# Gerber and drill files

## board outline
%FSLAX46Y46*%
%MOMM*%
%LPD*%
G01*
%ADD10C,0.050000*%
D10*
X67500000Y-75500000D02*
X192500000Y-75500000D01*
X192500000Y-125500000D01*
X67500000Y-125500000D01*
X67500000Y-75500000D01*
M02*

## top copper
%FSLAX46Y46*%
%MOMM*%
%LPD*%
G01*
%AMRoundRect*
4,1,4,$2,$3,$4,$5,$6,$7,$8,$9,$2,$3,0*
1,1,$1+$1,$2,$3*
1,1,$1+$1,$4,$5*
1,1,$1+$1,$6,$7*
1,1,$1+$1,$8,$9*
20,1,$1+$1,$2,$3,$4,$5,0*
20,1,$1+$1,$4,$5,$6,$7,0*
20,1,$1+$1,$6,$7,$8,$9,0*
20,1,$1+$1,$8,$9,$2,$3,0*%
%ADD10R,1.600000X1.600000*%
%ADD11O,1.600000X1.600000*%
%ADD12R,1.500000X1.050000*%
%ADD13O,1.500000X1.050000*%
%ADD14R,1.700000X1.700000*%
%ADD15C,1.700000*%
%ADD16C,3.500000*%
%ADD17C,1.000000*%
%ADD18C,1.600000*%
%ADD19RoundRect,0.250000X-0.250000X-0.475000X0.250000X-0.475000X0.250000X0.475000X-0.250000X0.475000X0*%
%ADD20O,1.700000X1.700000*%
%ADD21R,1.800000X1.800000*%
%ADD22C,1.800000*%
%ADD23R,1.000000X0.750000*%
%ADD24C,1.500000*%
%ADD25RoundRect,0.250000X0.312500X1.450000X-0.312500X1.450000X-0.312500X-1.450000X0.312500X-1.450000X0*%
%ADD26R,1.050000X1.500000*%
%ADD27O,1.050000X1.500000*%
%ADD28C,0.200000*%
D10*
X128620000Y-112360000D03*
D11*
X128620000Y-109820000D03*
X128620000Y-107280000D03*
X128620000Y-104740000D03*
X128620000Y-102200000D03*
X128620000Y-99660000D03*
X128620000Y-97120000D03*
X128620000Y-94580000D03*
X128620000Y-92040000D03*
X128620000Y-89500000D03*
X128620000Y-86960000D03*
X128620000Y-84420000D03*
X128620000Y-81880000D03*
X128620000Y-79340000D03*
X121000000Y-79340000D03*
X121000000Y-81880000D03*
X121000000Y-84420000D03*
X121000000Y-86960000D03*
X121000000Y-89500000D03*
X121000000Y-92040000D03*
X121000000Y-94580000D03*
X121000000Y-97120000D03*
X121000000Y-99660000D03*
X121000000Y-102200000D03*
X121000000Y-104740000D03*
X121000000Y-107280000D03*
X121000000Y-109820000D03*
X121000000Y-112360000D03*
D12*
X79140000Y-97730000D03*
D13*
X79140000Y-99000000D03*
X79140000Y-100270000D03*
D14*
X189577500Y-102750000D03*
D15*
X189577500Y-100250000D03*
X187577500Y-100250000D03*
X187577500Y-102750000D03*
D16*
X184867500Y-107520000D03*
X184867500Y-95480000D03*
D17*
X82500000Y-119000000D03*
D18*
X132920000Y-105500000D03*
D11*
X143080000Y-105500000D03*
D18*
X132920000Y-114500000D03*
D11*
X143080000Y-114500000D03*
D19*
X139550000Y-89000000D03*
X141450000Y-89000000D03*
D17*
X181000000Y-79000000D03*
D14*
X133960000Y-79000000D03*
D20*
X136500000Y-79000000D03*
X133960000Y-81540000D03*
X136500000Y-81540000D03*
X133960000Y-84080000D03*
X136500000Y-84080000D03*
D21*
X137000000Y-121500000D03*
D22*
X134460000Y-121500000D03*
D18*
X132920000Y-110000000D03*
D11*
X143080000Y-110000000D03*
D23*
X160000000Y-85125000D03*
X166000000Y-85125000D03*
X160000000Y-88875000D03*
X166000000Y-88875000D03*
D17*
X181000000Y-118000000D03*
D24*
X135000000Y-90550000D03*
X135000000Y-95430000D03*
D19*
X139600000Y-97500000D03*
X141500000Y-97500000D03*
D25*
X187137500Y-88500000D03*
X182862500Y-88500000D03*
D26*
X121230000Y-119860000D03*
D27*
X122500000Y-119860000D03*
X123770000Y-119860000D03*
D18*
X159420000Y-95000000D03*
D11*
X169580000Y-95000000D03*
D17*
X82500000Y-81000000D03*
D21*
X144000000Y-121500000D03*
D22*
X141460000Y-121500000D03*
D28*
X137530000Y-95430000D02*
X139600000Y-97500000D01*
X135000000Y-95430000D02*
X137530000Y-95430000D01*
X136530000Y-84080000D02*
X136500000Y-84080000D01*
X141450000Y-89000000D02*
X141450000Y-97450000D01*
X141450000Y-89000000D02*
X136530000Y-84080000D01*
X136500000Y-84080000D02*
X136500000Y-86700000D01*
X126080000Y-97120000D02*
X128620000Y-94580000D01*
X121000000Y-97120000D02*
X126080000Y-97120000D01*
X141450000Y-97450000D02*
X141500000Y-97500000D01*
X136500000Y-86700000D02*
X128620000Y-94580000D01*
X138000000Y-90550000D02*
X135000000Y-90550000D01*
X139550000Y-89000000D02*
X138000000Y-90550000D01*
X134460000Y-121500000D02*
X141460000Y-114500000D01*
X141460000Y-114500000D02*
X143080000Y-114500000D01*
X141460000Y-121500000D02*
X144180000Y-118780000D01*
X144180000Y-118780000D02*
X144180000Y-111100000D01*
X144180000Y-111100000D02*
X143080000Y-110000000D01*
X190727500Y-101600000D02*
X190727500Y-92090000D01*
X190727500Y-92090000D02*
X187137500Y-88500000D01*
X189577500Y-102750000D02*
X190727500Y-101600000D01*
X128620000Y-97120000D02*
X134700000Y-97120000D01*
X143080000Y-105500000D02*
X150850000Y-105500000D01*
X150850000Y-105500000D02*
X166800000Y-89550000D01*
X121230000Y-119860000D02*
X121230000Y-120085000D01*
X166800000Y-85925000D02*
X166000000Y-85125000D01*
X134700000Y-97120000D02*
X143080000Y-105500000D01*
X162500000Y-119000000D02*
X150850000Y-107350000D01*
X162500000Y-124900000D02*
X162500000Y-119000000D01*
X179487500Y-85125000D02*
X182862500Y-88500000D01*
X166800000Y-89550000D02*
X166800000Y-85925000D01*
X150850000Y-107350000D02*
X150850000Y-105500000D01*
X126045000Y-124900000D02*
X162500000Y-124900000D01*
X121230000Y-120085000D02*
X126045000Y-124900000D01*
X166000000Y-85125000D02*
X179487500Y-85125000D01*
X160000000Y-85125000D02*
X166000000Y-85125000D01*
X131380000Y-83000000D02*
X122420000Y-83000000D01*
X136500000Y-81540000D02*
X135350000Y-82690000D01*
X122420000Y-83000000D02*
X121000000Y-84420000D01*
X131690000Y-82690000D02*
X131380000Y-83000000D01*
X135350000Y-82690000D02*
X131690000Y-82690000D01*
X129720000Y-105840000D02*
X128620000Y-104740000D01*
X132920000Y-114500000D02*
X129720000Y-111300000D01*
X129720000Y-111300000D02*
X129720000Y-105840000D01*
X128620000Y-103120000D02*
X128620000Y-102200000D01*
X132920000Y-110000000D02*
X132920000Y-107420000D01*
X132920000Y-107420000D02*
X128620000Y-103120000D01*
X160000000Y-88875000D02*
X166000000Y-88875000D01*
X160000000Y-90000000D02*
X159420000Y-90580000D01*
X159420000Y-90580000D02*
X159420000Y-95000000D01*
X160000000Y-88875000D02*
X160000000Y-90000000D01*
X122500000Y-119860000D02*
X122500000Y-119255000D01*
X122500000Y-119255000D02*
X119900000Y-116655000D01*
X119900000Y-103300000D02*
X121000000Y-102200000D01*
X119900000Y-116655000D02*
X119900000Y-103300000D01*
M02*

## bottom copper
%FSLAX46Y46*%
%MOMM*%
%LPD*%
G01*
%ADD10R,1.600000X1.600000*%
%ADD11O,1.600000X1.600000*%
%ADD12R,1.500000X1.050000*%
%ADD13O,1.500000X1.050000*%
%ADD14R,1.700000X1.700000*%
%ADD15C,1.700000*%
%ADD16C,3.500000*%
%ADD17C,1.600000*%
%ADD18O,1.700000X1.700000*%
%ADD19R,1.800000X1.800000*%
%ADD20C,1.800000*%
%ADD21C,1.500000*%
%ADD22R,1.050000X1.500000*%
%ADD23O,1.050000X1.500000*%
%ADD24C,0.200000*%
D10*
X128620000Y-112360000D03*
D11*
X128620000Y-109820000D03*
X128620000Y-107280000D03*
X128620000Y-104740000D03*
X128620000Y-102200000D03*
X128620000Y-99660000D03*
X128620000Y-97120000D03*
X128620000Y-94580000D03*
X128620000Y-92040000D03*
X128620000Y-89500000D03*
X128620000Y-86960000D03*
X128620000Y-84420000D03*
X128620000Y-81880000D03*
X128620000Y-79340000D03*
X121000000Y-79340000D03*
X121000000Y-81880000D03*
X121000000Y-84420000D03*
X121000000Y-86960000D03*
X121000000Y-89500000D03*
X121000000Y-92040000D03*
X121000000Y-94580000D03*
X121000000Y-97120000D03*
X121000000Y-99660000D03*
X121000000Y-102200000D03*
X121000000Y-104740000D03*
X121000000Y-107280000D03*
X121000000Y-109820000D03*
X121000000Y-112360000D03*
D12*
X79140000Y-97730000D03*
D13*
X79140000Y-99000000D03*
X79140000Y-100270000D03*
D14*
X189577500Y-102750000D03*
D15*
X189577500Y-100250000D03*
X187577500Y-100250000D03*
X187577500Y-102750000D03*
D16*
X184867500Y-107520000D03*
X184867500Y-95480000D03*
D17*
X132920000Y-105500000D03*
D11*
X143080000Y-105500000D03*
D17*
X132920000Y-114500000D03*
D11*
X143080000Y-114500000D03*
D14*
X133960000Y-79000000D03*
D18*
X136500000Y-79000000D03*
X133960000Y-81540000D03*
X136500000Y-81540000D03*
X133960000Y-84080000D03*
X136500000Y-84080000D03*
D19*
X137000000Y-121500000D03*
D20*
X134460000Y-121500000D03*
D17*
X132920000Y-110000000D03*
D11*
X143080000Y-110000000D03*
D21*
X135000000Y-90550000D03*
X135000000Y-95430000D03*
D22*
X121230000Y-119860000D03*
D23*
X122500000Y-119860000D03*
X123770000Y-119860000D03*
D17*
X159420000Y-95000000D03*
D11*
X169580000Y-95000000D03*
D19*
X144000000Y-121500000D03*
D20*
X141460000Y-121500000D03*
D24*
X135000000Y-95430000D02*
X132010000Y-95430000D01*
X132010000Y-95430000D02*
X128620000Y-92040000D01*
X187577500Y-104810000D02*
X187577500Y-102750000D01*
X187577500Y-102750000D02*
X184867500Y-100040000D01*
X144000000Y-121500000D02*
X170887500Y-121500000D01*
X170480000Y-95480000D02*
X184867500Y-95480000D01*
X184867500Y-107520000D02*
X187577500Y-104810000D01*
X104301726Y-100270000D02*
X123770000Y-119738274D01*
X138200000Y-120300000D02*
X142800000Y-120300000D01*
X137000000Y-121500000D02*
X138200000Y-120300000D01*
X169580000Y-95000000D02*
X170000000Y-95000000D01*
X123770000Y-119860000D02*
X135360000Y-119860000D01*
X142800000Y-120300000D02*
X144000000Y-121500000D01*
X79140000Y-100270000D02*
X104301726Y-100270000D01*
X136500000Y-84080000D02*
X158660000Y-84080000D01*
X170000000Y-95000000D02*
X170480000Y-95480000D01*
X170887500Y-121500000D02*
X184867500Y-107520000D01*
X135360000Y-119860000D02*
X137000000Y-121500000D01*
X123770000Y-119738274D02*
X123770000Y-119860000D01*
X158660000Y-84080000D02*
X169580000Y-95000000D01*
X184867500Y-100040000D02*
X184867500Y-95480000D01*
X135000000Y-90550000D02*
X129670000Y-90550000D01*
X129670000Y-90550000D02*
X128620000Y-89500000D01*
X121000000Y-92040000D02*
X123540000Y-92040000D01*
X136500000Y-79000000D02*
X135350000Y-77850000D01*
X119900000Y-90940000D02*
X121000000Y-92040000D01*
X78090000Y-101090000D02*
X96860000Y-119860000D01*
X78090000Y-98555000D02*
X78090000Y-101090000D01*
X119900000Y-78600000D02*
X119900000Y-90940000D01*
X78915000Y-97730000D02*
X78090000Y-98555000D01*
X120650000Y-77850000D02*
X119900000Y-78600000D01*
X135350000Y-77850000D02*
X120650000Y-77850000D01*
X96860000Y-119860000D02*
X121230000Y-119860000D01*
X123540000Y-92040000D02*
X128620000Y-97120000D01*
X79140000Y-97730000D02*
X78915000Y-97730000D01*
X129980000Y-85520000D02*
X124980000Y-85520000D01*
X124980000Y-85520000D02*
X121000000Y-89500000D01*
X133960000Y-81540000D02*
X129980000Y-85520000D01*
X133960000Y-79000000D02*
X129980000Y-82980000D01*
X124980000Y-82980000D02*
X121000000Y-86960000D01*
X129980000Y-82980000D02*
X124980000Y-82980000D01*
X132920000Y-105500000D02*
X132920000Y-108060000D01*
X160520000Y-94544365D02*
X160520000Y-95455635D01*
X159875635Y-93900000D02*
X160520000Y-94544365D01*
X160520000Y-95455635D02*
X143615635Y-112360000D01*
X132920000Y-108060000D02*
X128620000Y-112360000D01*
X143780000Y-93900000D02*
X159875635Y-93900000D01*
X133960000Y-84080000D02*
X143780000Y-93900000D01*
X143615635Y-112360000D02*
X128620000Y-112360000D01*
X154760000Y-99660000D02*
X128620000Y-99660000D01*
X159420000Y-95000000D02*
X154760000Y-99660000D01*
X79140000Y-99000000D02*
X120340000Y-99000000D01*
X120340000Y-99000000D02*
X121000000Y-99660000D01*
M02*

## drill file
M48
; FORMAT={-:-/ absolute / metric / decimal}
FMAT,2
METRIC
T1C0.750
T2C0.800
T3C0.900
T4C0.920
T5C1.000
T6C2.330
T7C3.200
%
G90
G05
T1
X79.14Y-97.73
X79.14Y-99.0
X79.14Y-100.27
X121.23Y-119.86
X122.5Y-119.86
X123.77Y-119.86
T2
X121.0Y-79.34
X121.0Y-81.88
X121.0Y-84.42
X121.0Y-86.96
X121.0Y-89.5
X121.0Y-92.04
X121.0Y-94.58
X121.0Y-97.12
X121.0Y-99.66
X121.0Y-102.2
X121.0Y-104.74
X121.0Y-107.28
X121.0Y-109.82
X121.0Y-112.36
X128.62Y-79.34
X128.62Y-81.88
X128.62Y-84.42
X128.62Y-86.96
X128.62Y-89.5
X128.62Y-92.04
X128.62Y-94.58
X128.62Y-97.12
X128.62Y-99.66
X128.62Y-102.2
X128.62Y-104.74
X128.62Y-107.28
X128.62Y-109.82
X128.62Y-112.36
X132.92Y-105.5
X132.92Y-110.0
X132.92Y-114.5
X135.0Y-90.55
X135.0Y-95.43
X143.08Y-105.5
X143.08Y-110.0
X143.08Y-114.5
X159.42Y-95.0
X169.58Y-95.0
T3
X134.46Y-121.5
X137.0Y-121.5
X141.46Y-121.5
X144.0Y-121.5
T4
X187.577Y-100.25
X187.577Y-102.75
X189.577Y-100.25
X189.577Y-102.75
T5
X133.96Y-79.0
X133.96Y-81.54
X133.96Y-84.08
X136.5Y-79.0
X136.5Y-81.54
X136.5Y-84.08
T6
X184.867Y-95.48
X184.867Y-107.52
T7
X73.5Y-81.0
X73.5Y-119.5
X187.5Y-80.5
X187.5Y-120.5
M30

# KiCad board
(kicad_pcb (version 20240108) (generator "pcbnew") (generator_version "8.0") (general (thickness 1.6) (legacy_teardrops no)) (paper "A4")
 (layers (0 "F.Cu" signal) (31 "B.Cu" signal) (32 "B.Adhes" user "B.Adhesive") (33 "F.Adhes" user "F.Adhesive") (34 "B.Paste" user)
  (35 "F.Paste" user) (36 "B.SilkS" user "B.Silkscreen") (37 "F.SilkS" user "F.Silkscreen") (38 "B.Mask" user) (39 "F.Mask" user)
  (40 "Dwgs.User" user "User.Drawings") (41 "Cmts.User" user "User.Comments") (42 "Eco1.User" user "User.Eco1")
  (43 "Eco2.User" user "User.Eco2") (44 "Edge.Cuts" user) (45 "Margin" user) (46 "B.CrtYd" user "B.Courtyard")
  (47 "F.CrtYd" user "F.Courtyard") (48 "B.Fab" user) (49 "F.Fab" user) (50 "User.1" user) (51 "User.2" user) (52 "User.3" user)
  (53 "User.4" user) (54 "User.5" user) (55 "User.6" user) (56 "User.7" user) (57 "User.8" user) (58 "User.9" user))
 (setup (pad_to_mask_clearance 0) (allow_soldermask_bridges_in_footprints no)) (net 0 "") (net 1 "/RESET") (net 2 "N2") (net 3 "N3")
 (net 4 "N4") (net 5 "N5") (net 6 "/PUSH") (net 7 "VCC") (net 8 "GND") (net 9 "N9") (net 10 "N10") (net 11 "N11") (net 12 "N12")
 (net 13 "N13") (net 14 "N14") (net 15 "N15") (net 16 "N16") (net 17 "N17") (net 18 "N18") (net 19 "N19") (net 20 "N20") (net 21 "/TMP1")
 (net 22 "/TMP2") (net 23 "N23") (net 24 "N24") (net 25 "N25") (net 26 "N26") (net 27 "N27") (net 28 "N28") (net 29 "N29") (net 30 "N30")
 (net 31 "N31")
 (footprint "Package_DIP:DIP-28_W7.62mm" (layer "F.Cu") (at 128.62 112.36 180)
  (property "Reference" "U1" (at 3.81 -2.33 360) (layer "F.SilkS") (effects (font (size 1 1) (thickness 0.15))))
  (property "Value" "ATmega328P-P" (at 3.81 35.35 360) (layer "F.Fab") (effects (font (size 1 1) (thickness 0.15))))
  (pad "1" thru_hole rect (at 0 0 180) (size 1.6 1.6) (drill 0.8) (layers "*.Cu" "*.Mask") (remove_unused_layers no) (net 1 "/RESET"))
  (pad "2" thru_hole oval (at 0 2.54 180) (size 1.6 1.6) (drill 0.8) (layers "*.Cu" "*.Mask") (remove_unused_layers no) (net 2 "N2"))
  (pad "3" thru_hole oval (at 0 5.08 180) (size 1.6 1.6) (drill 0.8) (layers "*.Cu" "*.Mask") (remove_unused_layers no) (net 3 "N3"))
  (pad "4" thru_hole oval (at 0 7.62 180) (size 1.6 1.6) (drill 0.8) (layers "*.Cu" "*.Mask") (remove_unused_layers no) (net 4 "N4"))
  (pad "5" thru_hole oval (at 0 10.16 180) (size 1.6 1.6) (drill 0.8) (layers "*.Cu" "*.Mask") (remove_unused_layers no) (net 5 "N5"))
  (pad "6" thru_hole oval (at 0 12.7 180) (size 1.6 1.6) (drill 0.8) (layers "*.Cu" "*.Mask") (remove_unused_layers no) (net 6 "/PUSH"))
  (pad "7" thru_hole oval (at 0 15.24 180) (size 1.6 1.6) (drill 0.8) (layers "*.Cu" "*.Mask") (remove_unused_layers no) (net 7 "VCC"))
  (pad "8" thru_hole oval (at 0 17.78 180) (size 1.6 1.6) (drill 0.8) (layers "*.Cu" "*.Mask") (remove_unused_layers no) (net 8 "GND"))
  (pad "9" thru_hole oval (at 0 20.32 180) (size 1.6 1.6) (drill 0.8) (layers "*.Cu" "*.Mask") (remove_unused_layers no) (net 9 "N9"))
  (pad "10" thru_hole oval (at 0 22.86 180) (size 1.6 1.6) (drill 0.8) (layers "*.Cu" "*.Mask") (remove_unused_layers no) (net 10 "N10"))
  (pad "11" thru_hole oval (at 0 25.4 180) (size 1.6 1.6) (drill 0.8) (layers "*.Cu" "*.Mask") (remove_unused_layers no) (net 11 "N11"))
  (pad "12" thru_hole oval (at 0 27.94 180) (size 1.6 1.6) (drill 0.8) (layers "*.Cu" "*.Mask") (remove_unused_layers no) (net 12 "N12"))
  (pad "13" thru_hole oval (at 0 30.48 180) (size 1.6 1.6) (drill 0.8) (layers "*.Cu" "*.Mask") (remove_unused_layers no) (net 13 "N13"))
  (pad "14" thru_hole oval (at 0 33.02 180) (size 1.6 1.6) (drill 0.8) (layers "*.Cu" "*.Mask") (remove_unused_layers no) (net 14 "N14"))
  (pad "15" thru_hole oval (at 7.62 33.02 180) (size 1.6 1.6) (drill 0.8) (layers "*.Cu" "*.Mask") (remove_unused_layers no) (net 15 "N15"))
  (pad "16" thru_hole oval (at 7.62 30.48 180) (size 1.6 1.6) (drill 0.8) (layers "*.Cu" "*.Mask") (remove_unused_layers no) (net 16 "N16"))
  (pad "17" thru_hole oval (at 7.62 27.94 180) (size 1.6 1.6) (drill 0.8) (layers "*.Cu" "*.Mask") (remove_unused_layers no) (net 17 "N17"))
  (pad "18" thru_hole oval (at 7.62 25.4 180) (size 1.6 1.6) (drill 0.8) (layers "*.Cu" "*.Mask") (remove_unused_layers no) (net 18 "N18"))
  (pad "19" thru_hole oval (at 7.62 22.86 180) (size 1.6 1.6) (drill 0.8) (layers "*.Cu" "*.Mask") (remove_unused_layers no) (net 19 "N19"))
  (pad "20" thru_hole oval (at 7.62 20.32 180) (size 1.6 1.6) (drill 0.8) (layers "*.Cu" "*.Mask") (remove_unused_layers no) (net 7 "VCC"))
  (pad "21" thru_hole oval (at 7.62 17.78 180) (size 1.6 1.6) (drill 0.8) (layers "*.Cu" "*.Mask") (remove_unused_layers no) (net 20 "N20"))
  (pad "22" thru_hole oval (at 7.62 15.24 180) (size 1.6 1.6) (drill 0.8) (layers "*.Cu" "*.Mask") (remove_unused_layers no) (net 8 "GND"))
  (pad "23" thru_hole oval (at 7.62 12.7 180) (size 1.6 1.6) (drill 0.8) (layers "*.Cu" "*.Mask") (remove_unused_layers no) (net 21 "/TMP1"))
  (pad "24" thru_hole oval (at 7.62 10.16 180) (size 1.6 1.6) (drill 0.8) (layers "*.Cu" "*.Mask") (remove_unused_layers no)
   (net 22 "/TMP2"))
  (pad "25" thru_hole oval (at 7.62 7.62 180) (size 1.6 1.6) (drill 0.8) (layers "*.Cu" "*.Mask") (remove_unused_layers no) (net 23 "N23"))
  (pad "26" thru_hole oval (at 7.62 5.08 180) (size 1.6 1.6) (drill 0.8) (layers "*.Cu" "*.Mask") (remove_unused_layers no) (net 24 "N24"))
  (pad "27" thru_hole oval (at 7.62 2.54 180) (size 1.6 1.6) (drill 0.8) (layers "*.Cu" "*.Mask") (remove_unused_layers no) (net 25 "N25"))
  (pad "28" thru_hole oval (at 7.62 0 180) (size 1.6 1.6) (drill 0.8) (layers "*.Cu" "*.Mask") (remove_unused_layers no) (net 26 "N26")))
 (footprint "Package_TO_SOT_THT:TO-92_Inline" (layer "F.Cu") (at 79.14 97.73 -90)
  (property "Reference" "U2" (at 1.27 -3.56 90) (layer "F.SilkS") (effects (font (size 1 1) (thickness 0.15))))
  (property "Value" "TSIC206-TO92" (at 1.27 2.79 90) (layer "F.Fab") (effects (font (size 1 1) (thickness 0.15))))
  (pad "1" thru_hole rect (at 0 0 270) (size 1.05 1.5) (drill 0.75) (layers "*.Cu" "*.Mask") (remove_unused_layers no) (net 7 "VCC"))
  (pad "2" thru_hole oval (at 1.27 0 270) (size 1.05 1.5) (drill 0.75) (layers "*.Cu" "*.Mask") (remove_unused_layers no) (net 21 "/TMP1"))
  (pad "3" thru_hole oval (at 2.54 0 270) (size 1.05 1.5) (drill 0.75) (layers "*.Cu" "*.Mask") (remove_unused_layers no) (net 8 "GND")))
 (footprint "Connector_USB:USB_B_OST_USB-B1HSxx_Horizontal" (layer "F.Cu") (at 189.5775 102.75 180)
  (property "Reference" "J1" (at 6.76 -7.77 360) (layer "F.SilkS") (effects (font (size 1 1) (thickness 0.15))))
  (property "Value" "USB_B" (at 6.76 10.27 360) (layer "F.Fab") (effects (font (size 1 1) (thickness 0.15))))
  (pad "1" thru_hole rect (at 0 0 180) (size 1.7 1.7) (drill 0.92) (layers "*.Cu" "*.Mask") (remove_unused_layers no) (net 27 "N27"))
  (pad "2" thru_hole circle (at 0 2.5 180) (size 1.7 1.7) (drill 0.92) (layers "*.Cu" "*.Mask") (remove_unused_layers no) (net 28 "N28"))
  (pad "3" thru_hole circle (at 2 2.5 180) (size 1.7 1.7) (drill 0.92) (layers "*.Cu" "*.Mask") (remove_unused_layers no) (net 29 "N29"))
  (pad "4" thru_hole circle (at 2 0 180) (size 1.7 1.7) (drill 0.92) (layers "*.Cu" "*.Mask") (remove_unused_layers no) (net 8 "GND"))
  (pad "5" thru_hole circle (at 4.71 -4.77 180) (size 3.5 3.5) (drill 2.33) (layers "*.Cu" "*.Mask") (remove_unused_layers no) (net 8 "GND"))
  (pad "5" thru_hole circle (at 4.71 7.27 180) (size 3.5 3.5) (drill 2.33) (layers "*.Cu" "*.Mask") (remove_unused_layers no) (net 8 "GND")))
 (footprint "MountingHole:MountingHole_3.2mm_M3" (layer "F.Cu") (at 73.5 81)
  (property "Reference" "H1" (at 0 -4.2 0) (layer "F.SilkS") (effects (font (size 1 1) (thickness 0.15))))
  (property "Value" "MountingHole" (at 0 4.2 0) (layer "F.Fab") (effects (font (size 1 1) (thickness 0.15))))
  (pad "" np_thru_hole circle (at 0 0) (size 3.2 3.2) (drill 3.2) (layers "*.Cu" "*.Mask")))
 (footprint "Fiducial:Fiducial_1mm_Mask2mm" (layer "F.Cu") (at 82.5 119)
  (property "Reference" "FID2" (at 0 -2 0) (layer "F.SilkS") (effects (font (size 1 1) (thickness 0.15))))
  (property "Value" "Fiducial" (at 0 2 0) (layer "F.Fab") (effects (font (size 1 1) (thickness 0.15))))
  (pad "" smd circle (at 0 0) (size 1 1) (layers "F.Cu" "F.Mask") (solder_mask_margin 0.5) (clearance 0.5)))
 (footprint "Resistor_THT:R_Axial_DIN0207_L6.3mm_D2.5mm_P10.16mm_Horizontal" (layer "F.Cu") (at 132.92 105.5)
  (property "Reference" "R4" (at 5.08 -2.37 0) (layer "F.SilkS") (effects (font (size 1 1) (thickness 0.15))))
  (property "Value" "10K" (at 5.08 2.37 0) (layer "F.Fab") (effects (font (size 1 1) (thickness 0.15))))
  (pad "1" thru_hole circle (at 0 0) (size 1.6 1.6) (drill 0.8) (layers "*.Cu" "*.Mask") (remove_unused_layers no) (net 1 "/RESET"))
  (pad "2" thru_hole oval (at 10.16 0) (size 1.6 1.6) (drill 0.8) (layers "*.Cu" "*.Mask") (remove_unused_layers no) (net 7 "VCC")))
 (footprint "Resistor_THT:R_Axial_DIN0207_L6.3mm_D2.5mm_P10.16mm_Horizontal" (layer "F.Cu") (at 132.92 114.5)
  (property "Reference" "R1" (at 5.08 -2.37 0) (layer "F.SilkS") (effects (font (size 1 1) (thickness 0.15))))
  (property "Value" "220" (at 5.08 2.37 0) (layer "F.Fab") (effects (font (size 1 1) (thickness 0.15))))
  (pad "1" thru_hole circle (at 0 0) (size 1.6 1.6) (drill 0.8) (layers "*.Cu" "*.Mask") (remove_unused_layers no) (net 4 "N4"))
  (pad "2" thru_hole oval (at 10.16 0) (size 1.6 1.6) (drill 0.8) (layers "*.Cu" "*.Mask") (remove_unused_layers no) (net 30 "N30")))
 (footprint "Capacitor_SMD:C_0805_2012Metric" (layer "F.Cu") (at 140.5 89)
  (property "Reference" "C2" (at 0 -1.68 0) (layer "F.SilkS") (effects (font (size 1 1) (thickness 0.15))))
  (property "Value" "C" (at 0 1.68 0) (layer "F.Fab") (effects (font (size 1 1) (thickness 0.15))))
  (pad "1" smd roundrect (at -0.95 0) (size 1 1.45) (layers "F.Cu" "F.Paste" "F.Mask") (roundrect_rratio 0.25) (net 10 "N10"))
  (pad "2" smd roundrect (at 0.95 0) (size 1 1.45) (layers "F.Cu" "F.Paste" "F.Mask") (roundrect_rratio 0.25) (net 8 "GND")))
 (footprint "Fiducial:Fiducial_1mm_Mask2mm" (layer "F.Cu") (at 181 79)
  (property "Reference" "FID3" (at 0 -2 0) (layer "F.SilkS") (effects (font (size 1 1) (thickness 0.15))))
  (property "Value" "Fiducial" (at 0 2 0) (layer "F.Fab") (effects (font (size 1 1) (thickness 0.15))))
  (pad "" smd circle (at 0 0) (size 1 1) (layers "F.Cu" "F.Mask") (solder_mask_margin 0.5) (clearance 0.5)))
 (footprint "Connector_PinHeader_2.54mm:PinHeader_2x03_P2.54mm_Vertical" (layer "F.Cu") (at 133.96 79)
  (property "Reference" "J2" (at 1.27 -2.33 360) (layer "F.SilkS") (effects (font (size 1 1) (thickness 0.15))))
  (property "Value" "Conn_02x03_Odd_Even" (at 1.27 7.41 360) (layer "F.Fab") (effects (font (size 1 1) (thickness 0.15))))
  (pad "1" thru_hole rect (at 0 0) (size 1.7 1.7) (drill 1) (layers "*.Cu" "*.Mask") (remove_unused_layers no) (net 18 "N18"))
  (pad "2" thru_hole oval (at 2.54 0) (size 1.7 1.7) (drill 1) (layers "*.Cu" "*.Mask") (remove_unused_layers no) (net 7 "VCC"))
  (pad "3" thru_hole oval (at 0 2.54) (size 1.7 1.7) (drill 1) (layers "*.Cu" "*.Mask") (remove_unused_layers no) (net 19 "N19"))
  (pad "4" thru_hole oval (at 2.54 2.54) (size 1.7 1.7) (drill 1) (layers "*.Cu" "*.Mask") (remove_unused_layers no) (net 17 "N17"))
  (pad "5" thru_hole oval (at 0 5.08) (size 1.7 1.7) (drill 1) (layers "*.Cu" "*.Mask") (remove_unused_layers no) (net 1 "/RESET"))
  (pad "6" thru_hole oval (at 2.54 5.08) (size 1.7 1.7) (drill 1) (layers "*.Cu" "*.Mask") (remove_unused_layers no) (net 8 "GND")))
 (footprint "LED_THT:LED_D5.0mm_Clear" (layer "F.Cu") (at 137 121.5 180)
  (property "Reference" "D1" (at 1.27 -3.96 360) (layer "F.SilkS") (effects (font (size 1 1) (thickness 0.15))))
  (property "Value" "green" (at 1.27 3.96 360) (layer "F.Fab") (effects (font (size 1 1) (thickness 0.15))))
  (pad "1" thru_hole rect (at 0 0 180) (size 1.8 1.8) (drill 0.9) (layers "*.Cu" "*.Mask") (remove_unused_layers no) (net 8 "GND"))
  (pad "2" thru_hole circle (at 2.54 0 180) (size 1.8 1.8) (drill 0.9) (layers "*.Cu" "*.Mask") (remove_unused_layers no) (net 30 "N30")))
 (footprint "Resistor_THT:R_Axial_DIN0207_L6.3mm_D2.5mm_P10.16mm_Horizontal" (layer "F.Cu") (at 132.92 110)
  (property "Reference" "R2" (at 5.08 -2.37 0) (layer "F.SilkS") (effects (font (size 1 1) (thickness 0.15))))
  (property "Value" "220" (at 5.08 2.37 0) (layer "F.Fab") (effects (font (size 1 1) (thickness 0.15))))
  (pad "1" thru_hole circle (at 0 0) (size 1.6 1.6) (drill 0.8) (layers "*.Cu" "*.Mask") (remove_unused_layers no) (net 5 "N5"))
  (pad "2" thru_hole oval (at 10.16 0) (size 1.6 1.6) (drill 0.8) (layers "*.Cu" "*.Mask") (remove_unused_layers no) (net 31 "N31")))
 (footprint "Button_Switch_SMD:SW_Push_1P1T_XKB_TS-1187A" (layer "F.Cu") (at 163 87)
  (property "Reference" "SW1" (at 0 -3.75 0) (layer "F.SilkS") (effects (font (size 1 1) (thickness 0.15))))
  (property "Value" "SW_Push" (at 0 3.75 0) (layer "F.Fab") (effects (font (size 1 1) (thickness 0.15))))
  (pad "1" smd rect (at -3 -1.875) (size 1 0.75) (layers "F.Cu" "F.Paste" "F.Mask") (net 7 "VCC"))
  (pad "1" smd rect (at 3 -1.875) (size 1 0.75) (layers "F.Cu" "F.Paste" "F.Mask") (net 7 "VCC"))
  (pad "2" smd rect (at -3 1.875) (size 1 0.75) (layers "F.Cu" "F.Paste" "F.Mask") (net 6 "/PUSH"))
  (pad "2" smd rect (at 3 1.875) (size 1 0.75) (layers "F.Cu" "F.Paste" "F.Mask") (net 6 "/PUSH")))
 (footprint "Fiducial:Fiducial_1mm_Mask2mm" (layer "F.Cu") (at 181 118)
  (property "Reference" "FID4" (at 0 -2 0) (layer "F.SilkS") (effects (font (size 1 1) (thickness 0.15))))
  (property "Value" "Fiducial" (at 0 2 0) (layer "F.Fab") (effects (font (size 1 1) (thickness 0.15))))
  (pad "" smd circle (at 0 0) (size 1 1) (layers "F.Cu" "F.Mask") (solder_mask_margin 0.5) (clearance 0.5)))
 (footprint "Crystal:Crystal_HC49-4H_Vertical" (layer "F.Cu") (at 135 90.55 -90)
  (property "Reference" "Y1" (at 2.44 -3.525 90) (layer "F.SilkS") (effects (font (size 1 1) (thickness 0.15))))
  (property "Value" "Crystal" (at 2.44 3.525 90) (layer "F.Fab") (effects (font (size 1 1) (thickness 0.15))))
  (pad "1" thru_hole circle (at 0 0 270) (size 1.5 1.5) (drill 0.8) (layers "*.Cu" "*.Mask") (remove_unused_layers no) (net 10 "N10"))
  (pad "2" thru_hole circle (at 4.88 0 270) (size 1.5 1.5) (drill 0.8) (layers "*.Cu" "*.Mask") (remove_unused_layers no) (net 9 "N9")))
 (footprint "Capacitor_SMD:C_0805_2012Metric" (layer "F.Cu") (at 140.55 97.5)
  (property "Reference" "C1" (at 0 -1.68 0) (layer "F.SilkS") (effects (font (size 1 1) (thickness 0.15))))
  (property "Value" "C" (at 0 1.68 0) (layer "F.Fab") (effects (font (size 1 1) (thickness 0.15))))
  (pad "1" smd roundrect (at -0.95 0) (size 1 1.45) (layers "F.Cu" "F.Paste" "F.Mask") (roundrect_rratio 0.25) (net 9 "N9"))
  (pad "2" smd roundrect (at 0.95 0) (size 1 1.45) (layers "F.Cu" "F.Paste" "F.Mask") (roundrect_rratio 0.25) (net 8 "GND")))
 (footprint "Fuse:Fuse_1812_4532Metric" (layer "F.Cu") (at 185 88.5 180)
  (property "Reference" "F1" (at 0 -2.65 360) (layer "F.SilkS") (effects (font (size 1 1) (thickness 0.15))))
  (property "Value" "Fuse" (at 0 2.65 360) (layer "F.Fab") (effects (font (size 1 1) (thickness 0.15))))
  (pad "1" smd roundrect (at -2.1375 0 180) (size 1.125 3.4) (layers "F.Cu" "F.Paste" "F.Mask") (roundrect_rratio 0.222222) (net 27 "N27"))
  (pad "2" smd roundrect (at 2.1375 0 180) (size 1.125 3.4) (layers "F.Cu" "F.Paste" "F.Mask") (roundrect_rratio 0.222222) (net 7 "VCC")))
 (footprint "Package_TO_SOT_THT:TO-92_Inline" (layer "F.Cu") (at 121.23 119.86)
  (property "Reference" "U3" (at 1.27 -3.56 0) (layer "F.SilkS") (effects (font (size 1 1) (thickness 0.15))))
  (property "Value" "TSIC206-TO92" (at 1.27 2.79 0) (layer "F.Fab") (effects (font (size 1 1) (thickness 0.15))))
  (pad "1" thru_hole rect (at 0 0) (size 1.05 1.5) (drill 0.75) (layers "*.Cu" "*.Mask") (remove_unused_layers no) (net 7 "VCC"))
  (pad "2" thru_hole oval (at 1.27 0) (size 1.05 1.5) (drill 0.75) (layers "*.Cu" "*.Mask") (remove_unused_layers no) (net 22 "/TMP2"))
  (pad "3" thru_hole oval (at 2.54 0) (size 1.05 1.5) (drill 0.75) (layers "*.Cu" "*.Mask") (remove_unused_layers no) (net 8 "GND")))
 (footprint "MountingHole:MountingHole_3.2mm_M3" (layer "F.Cu") (at 73.5 119.5)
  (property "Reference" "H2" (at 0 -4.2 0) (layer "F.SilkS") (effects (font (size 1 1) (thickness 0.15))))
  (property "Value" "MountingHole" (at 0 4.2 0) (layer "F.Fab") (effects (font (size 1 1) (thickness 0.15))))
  (pad "" np_thru_hole circle (at 0 0) (size 3.2 3.2) (drill 3.2) (layers "*.Cu" "*.Mask")))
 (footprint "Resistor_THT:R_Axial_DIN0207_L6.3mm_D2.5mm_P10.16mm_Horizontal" (layer "F.Cu") (at 159.42 95)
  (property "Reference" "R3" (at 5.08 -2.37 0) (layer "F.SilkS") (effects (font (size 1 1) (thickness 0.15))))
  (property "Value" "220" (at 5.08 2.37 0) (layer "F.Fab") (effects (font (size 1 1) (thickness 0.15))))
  (pad "1" thru_hole circle (at 0 0) (size 1.6 1.6) (drill 0.8) (layers "*.Cu" "*.Mask") (remove_unused_layers no) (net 6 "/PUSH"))
  (pad "2" thru_hole oval (at 10.16 0) (size 1.6 1.6) (drill 0.8) (layers "*.Cu" "*.Mask") (remove_unused_layers no) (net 8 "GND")))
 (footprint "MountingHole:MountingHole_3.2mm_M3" (layer "F.Cu") (at 187.5 80.5)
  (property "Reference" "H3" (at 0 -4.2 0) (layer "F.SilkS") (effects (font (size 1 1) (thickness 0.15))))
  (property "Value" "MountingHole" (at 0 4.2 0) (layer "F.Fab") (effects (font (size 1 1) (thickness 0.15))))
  (pad "" np_thru_hole circle (at 0 0) (size 3.2 3.2) (drill 3.2) (layers "*.Cu" "*.Mask")))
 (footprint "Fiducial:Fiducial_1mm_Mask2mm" (layer "F.Cu") (at 82.5 81)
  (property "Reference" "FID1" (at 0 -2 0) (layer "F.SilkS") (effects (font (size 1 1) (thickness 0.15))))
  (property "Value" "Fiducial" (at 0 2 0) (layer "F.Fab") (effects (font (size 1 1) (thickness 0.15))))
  (pad "" smd circle (at 0 0) (size 1 1) (layers "F.Cu" "F.Mask") (solder_mask_margin 0.5) (clearance 0.5)))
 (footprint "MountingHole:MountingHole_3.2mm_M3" (layer "F.Cu") (at 187.5 120.5)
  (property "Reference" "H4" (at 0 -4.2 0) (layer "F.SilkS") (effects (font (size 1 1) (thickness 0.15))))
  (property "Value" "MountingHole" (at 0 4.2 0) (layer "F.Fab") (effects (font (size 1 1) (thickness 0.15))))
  (pad "" np_thru_hole circle (at 0 0) (size 3.2 3.2) (drill 3.2) (layers "*.Cu" "*.Mask")))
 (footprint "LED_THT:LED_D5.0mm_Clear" (layer "F.Cu") (at 144 121.5 180)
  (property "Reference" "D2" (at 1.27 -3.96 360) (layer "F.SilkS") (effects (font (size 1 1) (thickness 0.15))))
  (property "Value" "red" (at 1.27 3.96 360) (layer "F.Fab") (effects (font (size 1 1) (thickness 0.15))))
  (pad "1" thru_hole rect (at 0 0 180) (size 1.8 1.8) (drill 0.9) (layers "*.Cu" "*.Mask") (remove_unused_layers no) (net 8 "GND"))
  (pad "2" thru_hole circle (at 2.54 0 180) (size 1.8 1.8) (drill 0.9) (layers "*.Cu" "*.Mask") (remove_unused_layers no) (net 31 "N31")))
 (gr_rect (start 67.5 75.5) (end 192.5 125.5) (stroke (width 0.05) (type default)) (fill none) (layer "Edge.Cuts"))
 (segment (start 137.53 95.43) (end 139.6 97.5) (width 0.2) (layer "F.Cu") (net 9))
 (segment (start 135 95.43) (end 137.53 95.43) (width 0.2) (layer "F.Cu") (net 9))
 (segment (start 135 95.43) (end 132.01 95.43) (width 0.2) (layer "B.Cu") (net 9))
 (segment (start 132.01 95.43) (end 128.62 92.04) (width 0.2) (layer "B.Cu") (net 9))
 (segment (start 136.53 84.08) (end 136.5 84.08) (width 0.2) (layer "F.Cu") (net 8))
 (segment (start 141.45 89) (end 141.45 97.45) (width 0.2) (layer "F.Cu") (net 8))
 (segment (start 141.45 89) (end 136.53 84.08) (width 0.2) (layer "F.Cu") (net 8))
 (segment (start 136.5 84.08) (end 136.5 86.7) (width 0.2) (layer "F.Cu") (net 8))
 (segment (start 126.08 97.12) (end 128.62 94.58) (width 0.2) (layer "F.Cu") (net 8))
 (segment (start 121 97.12) (end 126.08 97.12) (width 0.2) (layer "F.Cu") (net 8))
 (segment (start 141.45 97.45) (end 141.5 97.5) (width 0.2) (layer "F.Cu") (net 8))
 (segment (start 136.5 86.7) (end 128.62 94.58) (width 0.2) (layer "F.Cu") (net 8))
 (segment (start 187.5775 104.81) (end 187.5775 102.75) (width 0.2) (layer "B.Cu") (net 8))
 (segment (start 187.5775 102.75) (end 184.8675 100.04) (width 0.2) (layer "B.Cu") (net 8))
 (segment (start 144 121.5) (end 170.8875 121.5) (width 0.2) (layer "B.Cu") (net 8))
 (segment (start 170.48 95.48) (end 184.8675 95.48) (width 0.2) (layer "B.Cu") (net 8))
 (segment (start 184.8675 107.52) (end 187.5775 104.81) (width 0.2) (layer "B.Cu") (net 8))
 (segment (start 104.301726 100.27) (end 123.77 119.738274) (width 0.2) (layer "B.Cu") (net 8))
 (segment (start 138.2 120.3) (end 142.8 120.3) (width 0.2) (layer "B.Cu") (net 8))
 (segment (start 137 121.5) (end 138.2 120.3) (width 0.2) (layer "B.Cu") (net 8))
 (segment (start 169.58 95) (end 170 95) (width 0.2) (layer "B.Cu") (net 8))
 (segment (start 123.77 119.86) (end 135.36 119.86) (width 0.2) (layer "B.Cu") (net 8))
 (segment (start 142.8 120.3) (end 144 121.5) (width 0.2) (layer "B.Cu") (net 8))
 (segment (start 79.14 100.27) (end 104.301726 100.27) (width 0.2) (layer "B.Cu") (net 8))
 (segment (start 136.5 84.08) (end 158.66 84.08) (width 0.2) (layer "B.Cu") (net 8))
 (segment (start 170 95) (end 170.48 95.48) (width 0.2) (layer "B.Cu") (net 8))
 (segment (start 170.8875 121.5) (end 184.8675 107.52) (width 0.2) (layer "B.Cu") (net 8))
 (segment (start 135.36 119.86) (end 137 121.5) (width 0.2) (layer "B.Cu") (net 8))
 (segment (start 123.77 119.738274) (end 123.77 119.86) (width 0.2) (layer "B.Cu") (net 8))
 (segment (start 158.66 84.08) (end 169.58 95) (width 0.2) (layer "B.Cu") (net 8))
 (segment (start 184.8675 100.04) (end 184.8675 95.48) (width 0.2) (layer "B.Cu") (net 8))
 (segment (start 138 90.55) (end 135 90.55) (width 0.2) (layer "F.Cu") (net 10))
 (segment (start 139.55 89) (end 138 90.55) (width 0.2) (layer "F.Cu") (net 10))
 (segment (start 135 90.55) (end 129.67 90.55) (width 0.2) (layer "B.Cu") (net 10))
 (segment (start 129.67 90.55) (end 128.62 89.5) (width 0.2) (layer "B.Cu") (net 10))
 (segment (start 134.46 121.5) (end 141.46 114.5) (width 0.2) (layer "F.Cu") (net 30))
 (segment (start 141.46 114.5) (end 143.08 114.5) (width 0.2) (layer "F.Cu") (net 30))
 (segment (start 141.46 121.5) (end 144.18 118.78) (width 0.2) (layer "F.Cu") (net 31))
 (segment (start 144.18 118.78) (end 144.18 111.1) (width 0.2) (layer "F.Cu") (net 31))
 (segment (start 144.18 111.1) (end 143.08 110) (width 0.2) (layer "F.Cu") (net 31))
 (segment (start 190.7275 101.6) (end 190.7275 92.09) (width 0.2) (layer "F.Cu") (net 27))
 (segment (start 190.7275 92.09) (end 187.1375 88.5) (width 0.2) (layer "F.Cu") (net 27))
 (segment (start 189.5775 102.75) (end 190.7275 101.6) (width 0.2) (layer "F.Cu") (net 27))
 (segment (start 128.62 97.12) (end 134.7 97.12) (width 0.2) (layer "F.Cu") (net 7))
 (segment (start 143.08 105.5) (end 150.85 105.5) (width 0.2) (layer "F.Cu") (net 7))
 (segment (start 150.85 105.5) (end 166.8 89.55) (width 0.2) (layer "F.Cu") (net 7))
 (segment (start 121.23 119.86) (end 121.23 120.085) (width 0.2) (layer "F.Cu") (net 7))
 (segment (start 166.8 85.925) (end 166 85.125) (width 0.2) (layer "F.Cu") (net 7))
 (segment (start 134.7 97.12) (end 143.08 105.5) (width 0.2) (layer "F.Cu") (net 7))
 (segment (start 162.5 119) (end 150.85 107.35) (width 0.2) (layer "F.Cu") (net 7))
 (segment (start 162.5 124.9) (end 162.5 119) (width 0.2) (layer "F.Cu") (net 7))
 (segment (start 179.4875 85.125) (end 182.8625 88.5) (width 0.2) (layer "F.Cu") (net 7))
 (segment (start 166.8 89.55) (end 166.8 85.925) (width 0.2) (layer "F.Cu") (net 7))
 (segment (start 150.85 107.35) (end 150.85 105.5) (width 0.2) (layer "F.Cu") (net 7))
 (segment (start 126.045 124.9) (end 162.5 124.9) (width 0.2) (layer "F.Cu") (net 7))
 (segment (start 121.23 120.085) (end 126.045 124.9) (width 0.2) (layer "F.Cu") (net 7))
 (segment (start 166 85.125) (end 179.4875 85.125) (width 0.2) (layer "F.Cu") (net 7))
 (segment (start 160 85.125) (end 166 85.125) (width 0.2) (layer "F.Cu") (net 7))
 (segment (start 121 92.04) (end 123.54 92.04) (width 0.2) (layer "B.Cu") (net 7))
 (segment (start 136.5 79) (end 135.35 77.85) (width 0.2) (layer "B.Cu") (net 7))
 (segment (start 119.9 90.94) (end 121 92.04) (width 0.2) (layer "B.Cu") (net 7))
 (segment (start 78.09 101.09) (end 96.86 119.86) (width 0.2) (layer "B.Cu") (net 7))
 (segment (start 78.09 98.555) (end 78.09 101.09) (width 0.2) (layer "B.Cu") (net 7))
 (segment (start 119.9 78.6) (end 119.9 90.94) (width 0.2) (layer "B.Cu") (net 7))
 (segment (start 78.915 97.73) (end 78.09 98.555) (width 0.2) (layer "B.Cu") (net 7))
 (segment (start 120.65 77.85) (end 119.9 78.6) (width 0.2) (layer "B.Cu") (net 7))
 (segment (start 135.35 77.85) (end 120.65 77.85) (width 0.2) (layer "B.Cu") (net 7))
 (segment (start 96.86 119.86) (end 121.23 119.86) (width 0.2) (layer "B.Cu") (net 7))
 (segment (start 123.54 92.04) (end 128.62 97.12) (width 0.2) (layer "B.Cu") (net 7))
 (segment (start 79.14 97.73) (end 78.915 97.73) (width 0.2) (layer "B.Cu") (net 7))
 (segment (start 131.38 83) (end 122.42 83) (width 0.2) (layer "F.Cu") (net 17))
 (segment (start 136.5 81.54) (end 135.35 82.69) (width 0.2) (layer "F.Cu") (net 17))
 (segment (start 122.42 83) (end 121 84.42) (width 0.2) (layer "F.Cu") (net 17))
 (segment (start 131.69 82.69) (end 131.38 83) (width 0.2) (layer "F.Cu") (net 17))
 (segment (start 135.35 82.69) (end 131.69 82.69) (width 0.2) (layer "F.Cu") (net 17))
 (segment (start 129.98 85.52) (end 124.98 85.52) (width 0.2) (layer "B.Cu") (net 19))
 (segment (start 124.98 85.52) (end 121 89.5) (width 0.2) (layer "B.Cu") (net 19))
 (segment (start 133.96 81.54) (end 129.98 85.52) (width 0.2) (layer "B.Cu") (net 19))
 (segment (start 133.96 79) (end 129.98 82.98) (width 0.2) (layer "B.Cu") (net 18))
 (segment (start 124.98 82.98) (end 121 86.96) (width 0.2) (layer "B.Cu") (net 18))
 (segment (start 129.98 82.98) (end 124.98 82.98) (width 0.2) (layer "B.Cu") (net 18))
 (segment (start 132.92 105.5) (end 132.92 108.06) (width 0.2) (layer "B.Cu") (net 1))
 (segment (start 160.52 94.544365) (end 160.52 95.455635) (width 0.2) (layer "B.Cu") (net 1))
 (segment (start 159.875635 93.9) (end 160.52 94.544365) (width 0.2) (layer "B.Cu") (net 1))
 (segment (start 160.52 95.455635) (end 143.615635 112.36) (width 0.2) (layer "B.Cu") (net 1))
 (segment (start 132.92 108.06) (end 128.62 112.36) (width 0.2) (layer "B.Cu") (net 1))
 (segment (start 143.78 93.9) (end 159.875635 93.9) (width 0.2) (layer "B.Cu") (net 1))
 (segment (start 133.96 84.08) (end 143.78 93.9) (width 0.2) (layer "B.Cu") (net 1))
 (segment (start 143.615635 112.36) (end 128.62 112.36) (width 0.2) (layer "B.Cu") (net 1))
 (segment (start 129.72 105.84) (end 128.62 104.74) (width 0.2) (layer "F.Cu") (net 4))
 (segment (start 132.92 114.5) (end 129.72 111.3) (width 0.2) (layer "F.Cu") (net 4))
 (segment (start 129.72 111.3) (end 129.72 105.84) (width 0.2) (layer "F.Cu") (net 4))
 (segment (start 128.62 103.12) (end 128.62 102.2) (width 0.2) (layer "F.Cu") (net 5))
 (segment (start 132.92 110) (end 132.92 107.42) (width 0.2) (layer "F.Cu") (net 5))
 (segment (start 132.92 107.42) (end 128.62 103.12) (width 0.2) (layer "F.Cu") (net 5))
 (segment (start 160 88.875) (end 166 88.875) (width 0.2) (layer "F.Cu") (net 6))
 (segment (start 160 90) (end 159.42 90.58) (width 0.2) (layer "F.Cu") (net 6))
 (segment (start 159.42 90.58) (end 159.42 95) (width 0.2) (layer "F.Cu") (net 6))
 (segment (start 160 88.875) (end 160 90) (width 0.2) (layer "F.Cu") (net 6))
 (segment (start 154.76 99.66) (end 128.62 99.66) (width 0.2) (layer "B.Cu") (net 6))
 (segment (start 159.42 95) (end 154.76 99.66) (width 0.2) (layer "B.Cu") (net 6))
 (segment (start 122.5 119.86) (end 122.5 119.255) (width 0.2) (layer "F.Cu") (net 22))
 (segment (start 122.5 119.255) (end 119.9 116.655) (width 0.2) (layer "F.Cu") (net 22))
 (segment (start 119.9 103.3) (end 121 102.2) (width 0.2) (layer "F.Cu") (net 22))
 (segment (start 119.9 116.655) (end 119.9 103.3) (width 0.2) (layer "F.Cu") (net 22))
 (segment (start 79.14 99) (end 120.34 99) (width 0.2) (layer "B.Cu") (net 21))
 (segment (start 120.34 99) (end 121 99.66) (width 0.2) (layer "B.Cu") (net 21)))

